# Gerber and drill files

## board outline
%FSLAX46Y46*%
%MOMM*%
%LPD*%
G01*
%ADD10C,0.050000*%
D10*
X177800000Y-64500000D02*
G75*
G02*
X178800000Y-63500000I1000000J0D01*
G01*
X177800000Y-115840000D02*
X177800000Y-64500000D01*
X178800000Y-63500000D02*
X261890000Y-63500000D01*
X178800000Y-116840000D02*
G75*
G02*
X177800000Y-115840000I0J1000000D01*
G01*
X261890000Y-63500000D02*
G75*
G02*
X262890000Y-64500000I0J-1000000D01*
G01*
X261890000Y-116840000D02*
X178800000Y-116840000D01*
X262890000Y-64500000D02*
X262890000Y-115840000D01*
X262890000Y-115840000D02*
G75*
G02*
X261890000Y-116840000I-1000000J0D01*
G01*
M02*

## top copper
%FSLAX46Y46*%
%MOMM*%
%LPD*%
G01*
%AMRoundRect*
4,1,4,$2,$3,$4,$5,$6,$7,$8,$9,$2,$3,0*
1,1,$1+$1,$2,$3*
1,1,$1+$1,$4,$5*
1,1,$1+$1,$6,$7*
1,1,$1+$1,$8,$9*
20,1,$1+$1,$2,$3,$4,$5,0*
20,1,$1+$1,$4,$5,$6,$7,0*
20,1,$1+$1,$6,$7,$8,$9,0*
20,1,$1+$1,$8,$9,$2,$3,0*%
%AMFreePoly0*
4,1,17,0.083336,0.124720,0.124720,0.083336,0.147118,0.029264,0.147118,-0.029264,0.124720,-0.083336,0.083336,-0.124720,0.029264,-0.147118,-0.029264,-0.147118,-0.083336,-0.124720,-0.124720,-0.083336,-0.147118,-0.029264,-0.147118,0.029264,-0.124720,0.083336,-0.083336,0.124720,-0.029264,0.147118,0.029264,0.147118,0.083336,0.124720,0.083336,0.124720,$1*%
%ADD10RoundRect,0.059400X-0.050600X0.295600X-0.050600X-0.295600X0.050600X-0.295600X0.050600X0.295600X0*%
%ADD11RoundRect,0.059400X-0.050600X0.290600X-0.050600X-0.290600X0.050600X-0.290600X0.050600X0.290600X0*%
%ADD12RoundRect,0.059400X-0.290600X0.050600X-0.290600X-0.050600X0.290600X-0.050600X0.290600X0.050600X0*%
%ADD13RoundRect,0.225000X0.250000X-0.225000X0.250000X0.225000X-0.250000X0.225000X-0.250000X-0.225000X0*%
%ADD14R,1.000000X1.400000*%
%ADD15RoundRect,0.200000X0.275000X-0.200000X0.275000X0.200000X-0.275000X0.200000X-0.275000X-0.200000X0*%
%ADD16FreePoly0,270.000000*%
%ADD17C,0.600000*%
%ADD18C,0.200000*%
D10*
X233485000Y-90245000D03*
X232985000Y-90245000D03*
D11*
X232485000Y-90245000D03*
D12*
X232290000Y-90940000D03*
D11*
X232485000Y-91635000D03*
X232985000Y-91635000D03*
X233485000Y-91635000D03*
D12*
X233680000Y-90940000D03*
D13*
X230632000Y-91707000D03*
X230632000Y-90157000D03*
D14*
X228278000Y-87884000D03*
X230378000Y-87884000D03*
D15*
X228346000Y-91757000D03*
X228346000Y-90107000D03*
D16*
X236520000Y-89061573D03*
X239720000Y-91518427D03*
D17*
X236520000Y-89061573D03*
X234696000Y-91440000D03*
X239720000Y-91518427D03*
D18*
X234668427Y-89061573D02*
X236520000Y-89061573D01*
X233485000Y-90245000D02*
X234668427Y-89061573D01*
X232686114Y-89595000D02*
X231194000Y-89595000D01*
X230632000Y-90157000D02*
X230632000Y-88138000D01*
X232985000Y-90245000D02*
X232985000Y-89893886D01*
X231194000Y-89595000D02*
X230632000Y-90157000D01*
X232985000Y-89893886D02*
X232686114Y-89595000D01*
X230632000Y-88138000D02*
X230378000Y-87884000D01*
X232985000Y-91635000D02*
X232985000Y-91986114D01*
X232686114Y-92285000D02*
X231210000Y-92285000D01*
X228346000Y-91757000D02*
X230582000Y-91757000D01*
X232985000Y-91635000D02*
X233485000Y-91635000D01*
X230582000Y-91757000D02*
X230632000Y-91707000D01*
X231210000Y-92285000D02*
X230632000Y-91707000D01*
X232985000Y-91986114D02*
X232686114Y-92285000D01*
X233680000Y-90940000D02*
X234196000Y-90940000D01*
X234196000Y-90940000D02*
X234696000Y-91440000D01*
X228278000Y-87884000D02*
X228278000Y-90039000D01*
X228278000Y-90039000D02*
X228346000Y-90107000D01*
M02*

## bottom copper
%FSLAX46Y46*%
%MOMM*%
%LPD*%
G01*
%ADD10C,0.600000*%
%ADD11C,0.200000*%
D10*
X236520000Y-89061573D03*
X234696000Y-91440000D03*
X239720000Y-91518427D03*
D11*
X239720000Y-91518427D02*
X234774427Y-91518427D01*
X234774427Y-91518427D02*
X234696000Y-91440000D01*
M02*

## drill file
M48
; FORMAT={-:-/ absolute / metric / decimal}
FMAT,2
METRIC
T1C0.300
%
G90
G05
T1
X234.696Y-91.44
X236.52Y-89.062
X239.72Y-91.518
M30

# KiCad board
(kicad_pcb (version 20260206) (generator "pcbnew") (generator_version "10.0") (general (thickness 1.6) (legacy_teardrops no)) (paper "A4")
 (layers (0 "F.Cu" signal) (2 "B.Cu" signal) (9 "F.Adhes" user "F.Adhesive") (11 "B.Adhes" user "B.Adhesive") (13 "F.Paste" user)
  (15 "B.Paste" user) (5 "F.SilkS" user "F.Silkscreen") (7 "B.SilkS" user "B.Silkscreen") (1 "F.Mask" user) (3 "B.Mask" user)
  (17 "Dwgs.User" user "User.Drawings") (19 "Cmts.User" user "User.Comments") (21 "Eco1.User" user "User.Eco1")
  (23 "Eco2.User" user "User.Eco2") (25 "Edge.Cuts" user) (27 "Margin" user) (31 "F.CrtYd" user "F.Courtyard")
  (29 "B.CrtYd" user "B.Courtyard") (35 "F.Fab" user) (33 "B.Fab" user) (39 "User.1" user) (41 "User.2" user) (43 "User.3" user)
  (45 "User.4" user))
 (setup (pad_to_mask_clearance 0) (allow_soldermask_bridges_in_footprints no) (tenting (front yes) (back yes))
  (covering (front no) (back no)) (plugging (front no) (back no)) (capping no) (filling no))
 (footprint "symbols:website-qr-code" (layer "F.Cu") (at 184.15 110.49)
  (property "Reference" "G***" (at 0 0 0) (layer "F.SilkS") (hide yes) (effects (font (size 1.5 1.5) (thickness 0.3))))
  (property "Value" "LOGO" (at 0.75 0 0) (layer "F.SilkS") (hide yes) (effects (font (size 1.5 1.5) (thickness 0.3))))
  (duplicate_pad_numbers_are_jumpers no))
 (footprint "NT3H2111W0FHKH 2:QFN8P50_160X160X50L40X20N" (layer "F.Cu") (at 232.985 90.94 -90)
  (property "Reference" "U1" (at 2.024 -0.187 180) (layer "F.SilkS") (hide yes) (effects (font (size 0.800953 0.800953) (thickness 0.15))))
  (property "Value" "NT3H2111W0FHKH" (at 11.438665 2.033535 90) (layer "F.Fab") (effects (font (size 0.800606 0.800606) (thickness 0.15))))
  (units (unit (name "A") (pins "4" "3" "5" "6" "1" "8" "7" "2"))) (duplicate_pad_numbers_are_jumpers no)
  (pad "1" smd roundrect (at -0.695 -0.5 270) (size 0.71 0.22) (layers "F.Cu" "F.Mask" "F.Paste") (roundrect_rratio 0.27)
   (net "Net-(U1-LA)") (solder_mask_margin 0.102))
  (pad "2" smd roundrect (at -0.695 0 270) (size 0.71 0.22) (layers "F.Cu" "F.Mask" "F.Paste") (roundrect_rratio 0.27) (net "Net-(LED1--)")
   (solder_mask_margin 0.102))
  (pad "3" smd roundrect (at -0.695 0.5 270) (size 0.7 0.22) (layers "F.Cu" "F.Mask" "F.Paste") (roundrect_rratio 0.27)
   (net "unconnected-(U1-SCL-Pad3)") (solder_mask_margin 0.102))
  (pad "4" smd roundrect (at 0 0.695 270) (size 0.22 0.7) (layers "F.Cu" "F.Mask" "F.Paste") (roundrect_rratio 0.27)
   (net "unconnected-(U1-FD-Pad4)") (solder_mask_margin 0.102))
  (pad "5" smd roundrect (at 0.695 0.5 270) (size 0.7 0.22) (layers "F.Cu" "F.Mask" "F.Paste") (roundrect_rratio 0.27)
   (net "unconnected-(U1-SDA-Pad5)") (solder_mask_margin 0.102))
  (pad "6" smd roundrect (at 0.695 0 270) (size 0.7 0.22) (layers "F.Cu" "F.Mask" "F.Paste") (roundrect_rratio 0.27) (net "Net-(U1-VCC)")
   (solder_mask_margin 0.102))
  (pad "7" smd roundrect (at 0.695 -0.5 270) (size 0.7 0.22) (layers "F.Cu" "F.Mask" "F.Paste") (roundrect_rratio 0.27) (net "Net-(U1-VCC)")
   (solder_mask_margin 0.102))
  (pad "8" smd roundrect (at 0 -0.695 270) (size 0.22 0.7) (layers "F.Cu" "F.Mask" "F.Paste") (roundrect_rratio 0.27) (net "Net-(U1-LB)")
   (solder_mask_margin 0.102)))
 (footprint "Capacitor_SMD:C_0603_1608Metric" (layer "F.Cu") (at 230.632 90.932 90)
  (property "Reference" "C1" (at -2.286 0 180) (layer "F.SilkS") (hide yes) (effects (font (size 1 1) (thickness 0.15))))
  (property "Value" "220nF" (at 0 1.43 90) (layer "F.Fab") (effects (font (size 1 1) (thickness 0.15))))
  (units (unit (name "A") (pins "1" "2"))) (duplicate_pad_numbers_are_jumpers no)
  (pad "1" smd roundrect (at -0.775 0 90) (size 0.9 0.95) (layers "F.Cu" "F.Mask" "F.Paste") (roundrect_rratio 0.25) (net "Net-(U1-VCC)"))
  (pad "2" smd roundrect (at 0.775 0 90) (size 0.9 0.95) (layers "F.Cu" "F.Mask" "F.Paste") (roundrect_rratio 0.25) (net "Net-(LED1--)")))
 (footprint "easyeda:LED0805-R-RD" (layer "F.Cu") (at 229.328 87.884 180)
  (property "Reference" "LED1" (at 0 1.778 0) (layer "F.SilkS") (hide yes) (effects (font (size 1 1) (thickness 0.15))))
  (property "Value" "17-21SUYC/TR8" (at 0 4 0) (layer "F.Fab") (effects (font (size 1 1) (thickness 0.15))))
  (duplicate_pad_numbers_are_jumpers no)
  (pad "1" smd rect (at 1.05 0) (size 1 1.4) (layers "F.Cu" "F.Mask" "F.Paste") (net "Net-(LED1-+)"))
  (pad "2" smd rect (at -1.05 0) (size 1 1.4) (layers "F.Cu" "F.Mask" "F.Paste") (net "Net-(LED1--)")))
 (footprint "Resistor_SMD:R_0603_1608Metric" (layer "F.Cu") (at 228.346 90.932 90)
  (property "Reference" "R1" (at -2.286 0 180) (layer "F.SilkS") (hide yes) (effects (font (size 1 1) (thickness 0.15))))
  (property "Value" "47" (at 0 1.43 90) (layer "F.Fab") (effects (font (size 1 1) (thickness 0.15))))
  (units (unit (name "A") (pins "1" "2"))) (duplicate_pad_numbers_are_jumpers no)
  (pad "1" smd roundrect (at -0.825 0 90) (size 0.8 0.95) (layers "F.Cu" "F.Mask" "F.Paste") (roundrect_rratio 0.25) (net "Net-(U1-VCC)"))
  (pad "2" smd roundrect (at 0.825 0 90) (size 0.8 0.95) (layers "F.Cu" "F.Mask" "F.Paste") (roundrect_rratio 0.25) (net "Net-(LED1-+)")))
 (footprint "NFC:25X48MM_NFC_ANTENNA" (layer "F.Cu") (at 261.37 66.29 -90)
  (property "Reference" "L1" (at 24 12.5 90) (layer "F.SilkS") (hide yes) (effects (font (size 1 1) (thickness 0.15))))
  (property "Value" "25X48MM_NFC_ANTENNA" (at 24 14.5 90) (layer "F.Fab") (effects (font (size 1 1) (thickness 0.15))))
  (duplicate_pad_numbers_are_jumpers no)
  (pad "1" smd custom (at 22.771573 24.85 270) (size 0.3 0.3) (layers "F.Cu") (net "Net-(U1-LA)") (zone_connect 0) (thermal_bridge_angle 90)
   (options (clearance outline) (anchor circle)) (primitives))
  (pad "2" smd custom (at 25.228427 21.65 270) (size 0.3 0.3) (layers "F.Cu") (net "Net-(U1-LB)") (zone_connect 0) (thermal_bridge_angle 90)
   (options (clearance outline) (anchor circle)) (primitives)))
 (gr_arc (start 177.8 64.5) (mid 178.092893 63.792893) (end 178.8 63.5) (stroke (width 0.05) (type default)) (layer "Edge.Cuts"))
 (gr_line (start 177.8 115.84) (end 177.8 64.5) (stroke (width 0.05) (type default)) (layer "Edge.Cuts"))
 (gr_line (start 178.8 63.5) (end 261.89 63.5) (stroke (width 0.05) (type default)) (layer "Edge.Cuts"))
 (gr_arc (start 178.8 116.84) (mid 178.092893 116.547107) (end 177.8 115.84) (stroke (width 0.05) (type default)) (layer "Edge.Cuts"))
 (gr_arc (start 261.89 63.5) (mid 262.597107 63.792893) (end 262.89 64.5) (stroke (width 0.05) (type default)) (layer "Edge.Cuts"))
 (gr_line (start 261.89 116.84) (end 178.8 116.84) (stroke (width 0.05) (type default)) (layer "Edge.Cuts"))
 (gr_line (start 262.89 64.5) (end 262.89 115.84) (stroke (width 0.05) (type default)) (layer "Edge.Cuts"))
 (gr_arc (start 262.89 115.84) (mid 262.597107 116.547107) (end 261.89 116.84) (stroke (width 0.05) (type default)) (layer "Edge.Cuts"))
 (segment (start 234.668427 89.061573) (end 236.52 89.061573) (width 0.2) (layer "F.Cu") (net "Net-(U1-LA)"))
 (segment (start 233.485 90.245) (end 234.668427 89.061573) (width 0.2) (layer "F.Cu") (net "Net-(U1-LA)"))
 (via (at 236.52 89.061573) (size 0.6) (drill 0.3) (layers "F.Cu" "B.Cu") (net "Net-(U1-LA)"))
 (segment (start 232.686114 89.595) (end 231.194 89.595) (width 0.2) (layer "F.Cu") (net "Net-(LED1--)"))
 (segment (start 230.632 90.157) (end 230.632 88.138) (width 0.2) (layer "F.Cu") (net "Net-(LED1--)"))
 (segment (start 232.985 90.245) (end 232.985 89.893886) (width 0.2) (layer "F.Cu") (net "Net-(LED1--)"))
 (segment (start 231.194 89.595) (end 230.632 90.157) (width 0.2) (layer "F.Cu") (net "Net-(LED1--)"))
 (segment (start 232.985 89.893886) (end 232.686114 89.595) (width 0.2) (layer "F.Cu") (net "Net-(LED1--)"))
 (segment (start 230.632 88.138) (end 230.378 87.884) (width 0.2) (layer "F.Cu") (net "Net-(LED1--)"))
 (segment (start 232.985 91.635) (end 232.985 91.986114) (width 0.2) (layer "F.Cu") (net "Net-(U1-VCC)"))
 (segment (start 232.686114 92.285) (end 231.21 92.285) (width 0.2) (layer "F.Cu") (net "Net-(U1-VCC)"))
 (segment (start 228.346 91.757) (end 230.582 91.757) (width 0.2) (layer "F.Cu") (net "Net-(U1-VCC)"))
 (segment (start 232.985 91.635) (end 233.485 91.635) (width 0.2) (layer "F.Cu") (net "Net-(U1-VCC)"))
 (segment (start 230.582 91.757) (end 230.632 91.707) (width 0.2) (layer "F.Cu") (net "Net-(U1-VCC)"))
 (segment (start 231.21 92.285) (end 230.632 91.707) (width 0.2) (layer "F.Cu") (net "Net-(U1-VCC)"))
 (segment (start 232.985 91.986114) (end 232.686114 92.285) (width 0.2) (layer "F.Cu") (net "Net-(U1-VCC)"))
 (segment (start 233.68 90.94) (end 234.196 90.94) (width 0.2) (layer "F.Cu") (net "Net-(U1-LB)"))
 (segment (start 234.196 90.94) (end 234.696 91.44) (width 0.2) (layer "F.Cu") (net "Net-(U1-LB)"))
 (via (at 234.696 91.44) (size 0.6) (drill 0.3) (layers "F.Cu" "B.Cu") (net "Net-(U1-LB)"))
 (via (at 239.72 91.518427) (size 0.6) (drill 0.3) (layers "F.Cu" "B.Cu") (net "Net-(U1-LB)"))
 (segment (start 239.72 91.518427) (end 234.774427 91.518427) (width 0.2) (layer "B.Cu") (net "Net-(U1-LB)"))
 (segment (start 234.774427 91.518427) (end 234.696 91.44) (width 0.2) (layer "B.Cu") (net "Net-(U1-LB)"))
 (segment (start 228.278 87.884) (end 228.278 90.039) (width 0.2) (layer "F.Cu") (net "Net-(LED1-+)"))
 (segment (start 228.278 90.039) (end 228.346 90.107) (width 0.2) (layer "F.Cu") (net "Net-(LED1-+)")))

